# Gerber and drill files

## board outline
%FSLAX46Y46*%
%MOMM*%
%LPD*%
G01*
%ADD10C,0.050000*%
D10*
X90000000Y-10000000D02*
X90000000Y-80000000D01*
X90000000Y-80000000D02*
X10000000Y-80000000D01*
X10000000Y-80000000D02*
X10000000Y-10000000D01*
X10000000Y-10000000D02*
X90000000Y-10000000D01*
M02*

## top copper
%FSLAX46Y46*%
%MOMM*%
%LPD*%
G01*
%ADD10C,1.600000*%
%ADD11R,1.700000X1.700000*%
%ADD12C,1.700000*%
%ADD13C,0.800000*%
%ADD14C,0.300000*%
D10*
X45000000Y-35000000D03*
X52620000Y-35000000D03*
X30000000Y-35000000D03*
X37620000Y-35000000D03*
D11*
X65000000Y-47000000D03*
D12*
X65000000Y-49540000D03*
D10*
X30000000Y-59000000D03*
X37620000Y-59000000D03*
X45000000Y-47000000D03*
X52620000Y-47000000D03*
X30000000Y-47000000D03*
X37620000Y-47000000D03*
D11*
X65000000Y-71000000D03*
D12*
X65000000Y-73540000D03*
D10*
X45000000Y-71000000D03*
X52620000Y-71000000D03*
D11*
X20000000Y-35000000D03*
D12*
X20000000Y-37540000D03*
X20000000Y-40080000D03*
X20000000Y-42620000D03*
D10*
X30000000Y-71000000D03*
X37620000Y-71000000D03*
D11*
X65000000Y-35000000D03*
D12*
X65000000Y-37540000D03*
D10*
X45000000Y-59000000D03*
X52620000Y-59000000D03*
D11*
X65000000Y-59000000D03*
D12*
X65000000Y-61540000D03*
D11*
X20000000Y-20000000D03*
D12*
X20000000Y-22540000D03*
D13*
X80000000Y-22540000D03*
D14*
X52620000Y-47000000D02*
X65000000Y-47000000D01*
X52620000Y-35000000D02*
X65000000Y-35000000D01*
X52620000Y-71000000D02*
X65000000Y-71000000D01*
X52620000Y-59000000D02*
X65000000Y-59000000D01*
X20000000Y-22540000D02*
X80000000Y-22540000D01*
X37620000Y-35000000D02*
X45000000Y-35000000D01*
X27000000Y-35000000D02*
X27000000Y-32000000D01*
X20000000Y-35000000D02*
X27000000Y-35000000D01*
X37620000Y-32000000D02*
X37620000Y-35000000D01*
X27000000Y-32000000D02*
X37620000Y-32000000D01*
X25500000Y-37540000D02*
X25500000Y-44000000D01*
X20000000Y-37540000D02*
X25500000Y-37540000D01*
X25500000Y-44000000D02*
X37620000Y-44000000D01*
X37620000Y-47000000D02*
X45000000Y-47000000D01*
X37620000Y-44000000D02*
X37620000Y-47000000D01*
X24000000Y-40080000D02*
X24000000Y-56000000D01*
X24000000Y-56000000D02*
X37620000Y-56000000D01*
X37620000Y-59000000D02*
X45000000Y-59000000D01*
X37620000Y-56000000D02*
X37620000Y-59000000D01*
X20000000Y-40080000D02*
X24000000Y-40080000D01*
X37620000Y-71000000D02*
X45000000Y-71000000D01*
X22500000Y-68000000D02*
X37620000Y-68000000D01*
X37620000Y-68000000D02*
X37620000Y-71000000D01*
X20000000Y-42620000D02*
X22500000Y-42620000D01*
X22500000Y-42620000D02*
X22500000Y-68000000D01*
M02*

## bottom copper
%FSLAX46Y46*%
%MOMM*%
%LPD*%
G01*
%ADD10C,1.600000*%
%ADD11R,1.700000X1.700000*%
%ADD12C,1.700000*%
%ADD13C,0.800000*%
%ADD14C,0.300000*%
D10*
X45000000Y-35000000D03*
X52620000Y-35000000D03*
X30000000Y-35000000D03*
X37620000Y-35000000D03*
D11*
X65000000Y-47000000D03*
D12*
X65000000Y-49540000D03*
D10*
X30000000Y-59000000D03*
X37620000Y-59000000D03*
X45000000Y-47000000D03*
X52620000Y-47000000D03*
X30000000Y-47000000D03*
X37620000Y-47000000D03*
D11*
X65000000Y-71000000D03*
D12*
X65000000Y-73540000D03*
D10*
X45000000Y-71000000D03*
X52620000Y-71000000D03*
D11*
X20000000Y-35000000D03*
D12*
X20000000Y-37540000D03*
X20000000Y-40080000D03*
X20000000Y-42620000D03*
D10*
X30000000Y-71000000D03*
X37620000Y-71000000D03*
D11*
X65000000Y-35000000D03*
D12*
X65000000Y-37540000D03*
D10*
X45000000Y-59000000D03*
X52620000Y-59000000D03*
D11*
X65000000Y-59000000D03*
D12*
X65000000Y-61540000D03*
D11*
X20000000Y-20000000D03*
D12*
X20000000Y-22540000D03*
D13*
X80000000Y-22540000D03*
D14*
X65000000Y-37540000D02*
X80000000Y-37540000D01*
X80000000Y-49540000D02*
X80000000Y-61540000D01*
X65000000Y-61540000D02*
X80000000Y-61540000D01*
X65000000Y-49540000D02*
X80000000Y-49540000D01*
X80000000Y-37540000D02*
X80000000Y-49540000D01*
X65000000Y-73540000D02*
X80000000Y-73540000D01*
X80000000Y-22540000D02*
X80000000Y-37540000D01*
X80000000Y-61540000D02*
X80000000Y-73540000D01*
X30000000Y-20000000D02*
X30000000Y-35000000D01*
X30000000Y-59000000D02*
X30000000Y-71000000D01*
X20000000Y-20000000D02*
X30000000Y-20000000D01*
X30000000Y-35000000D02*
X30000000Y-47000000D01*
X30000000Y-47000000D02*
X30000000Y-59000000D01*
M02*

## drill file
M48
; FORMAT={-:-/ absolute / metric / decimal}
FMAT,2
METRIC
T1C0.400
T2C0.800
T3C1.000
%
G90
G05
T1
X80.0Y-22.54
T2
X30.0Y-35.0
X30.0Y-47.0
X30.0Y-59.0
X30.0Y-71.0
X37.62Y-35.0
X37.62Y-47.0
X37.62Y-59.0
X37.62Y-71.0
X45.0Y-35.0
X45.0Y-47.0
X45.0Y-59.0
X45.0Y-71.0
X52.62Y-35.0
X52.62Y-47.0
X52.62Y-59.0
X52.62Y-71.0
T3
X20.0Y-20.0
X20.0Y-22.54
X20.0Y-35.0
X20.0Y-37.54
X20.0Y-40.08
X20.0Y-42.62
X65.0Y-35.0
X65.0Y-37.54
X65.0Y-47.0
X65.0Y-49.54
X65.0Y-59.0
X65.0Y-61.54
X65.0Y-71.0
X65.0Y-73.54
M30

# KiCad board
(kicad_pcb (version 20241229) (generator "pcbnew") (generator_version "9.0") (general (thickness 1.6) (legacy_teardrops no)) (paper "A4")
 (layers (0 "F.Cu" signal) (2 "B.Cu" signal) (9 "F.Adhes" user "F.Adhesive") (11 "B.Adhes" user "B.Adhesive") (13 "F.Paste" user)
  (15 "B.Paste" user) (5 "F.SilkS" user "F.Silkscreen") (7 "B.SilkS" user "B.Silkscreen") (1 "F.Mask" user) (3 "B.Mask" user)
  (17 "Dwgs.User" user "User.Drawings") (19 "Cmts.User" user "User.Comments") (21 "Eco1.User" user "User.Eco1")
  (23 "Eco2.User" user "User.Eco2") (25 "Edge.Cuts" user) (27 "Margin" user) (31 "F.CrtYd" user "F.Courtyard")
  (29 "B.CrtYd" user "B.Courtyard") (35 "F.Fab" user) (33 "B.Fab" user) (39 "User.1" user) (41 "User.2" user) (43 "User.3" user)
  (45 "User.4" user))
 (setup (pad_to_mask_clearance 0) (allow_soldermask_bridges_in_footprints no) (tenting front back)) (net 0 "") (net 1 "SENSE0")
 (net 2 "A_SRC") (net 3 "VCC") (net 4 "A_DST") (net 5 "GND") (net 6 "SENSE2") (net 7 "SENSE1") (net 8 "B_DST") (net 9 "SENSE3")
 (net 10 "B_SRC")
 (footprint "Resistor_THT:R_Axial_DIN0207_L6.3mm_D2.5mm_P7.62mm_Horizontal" (layer "F.Cu") (at 45 35)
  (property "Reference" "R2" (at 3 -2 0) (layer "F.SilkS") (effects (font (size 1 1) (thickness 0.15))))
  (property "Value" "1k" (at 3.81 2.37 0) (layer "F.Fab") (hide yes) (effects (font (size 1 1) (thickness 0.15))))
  (pad "1" thru_hole circle (at 0 0) (size 1.6 1.6) (drill 0.8) (layers "*.Cu" "*.Mask") (remove_unused_layers no) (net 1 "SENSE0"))
  (pad "2" thru_hole circle (at 7.62 0) (size 1.6 1.6) (drill 0.8) (layers "*.Cu" "*.Mask") (remove_unused_layers no) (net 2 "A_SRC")))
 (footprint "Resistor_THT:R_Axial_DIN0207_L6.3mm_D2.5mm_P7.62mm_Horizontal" (layer "F.Cu") (at 30 35)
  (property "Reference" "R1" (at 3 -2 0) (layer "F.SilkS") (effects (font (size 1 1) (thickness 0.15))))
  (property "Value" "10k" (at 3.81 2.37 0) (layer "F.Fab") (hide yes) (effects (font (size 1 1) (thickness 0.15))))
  (pad "1" thru_hole circle (at 0 0) (size 1.6 1.6) (drill 0.8) (layers "*.Cu" "*.Mask") (remove_unused_layers no) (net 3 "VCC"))
  (pad "2" thru_hole circle (at 7.62 0) (size 1.6 1.6) (drill 0.8) (layers "*.Cu" "*.Mask") (remove_unused_layers no) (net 1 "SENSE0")))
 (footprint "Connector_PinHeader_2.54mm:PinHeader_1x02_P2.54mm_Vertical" (layer "F.Cu") (at 65 47)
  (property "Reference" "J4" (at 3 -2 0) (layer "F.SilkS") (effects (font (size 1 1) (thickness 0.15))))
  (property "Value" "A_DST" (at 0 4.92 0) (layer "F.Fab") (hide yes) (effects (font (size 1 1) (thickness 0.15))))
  (pad "1" thru_hole rect (at 0 0) (size 1.7 1.7) (drill 1) (layers "*.Cu" "*.Mask") (remove_unused_layers no) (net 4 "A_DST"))
  (pad "2" thru_hole circle (at 0 2.54) (size 1.7 1.7) (drill 1) (layers "*.Cu" "*.Mask") (remove_unused_layers no) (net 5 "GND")))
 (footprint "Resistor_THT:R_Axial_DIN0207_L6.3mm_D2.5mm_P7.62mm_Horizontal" (layer "F.Cu") (at 30 59)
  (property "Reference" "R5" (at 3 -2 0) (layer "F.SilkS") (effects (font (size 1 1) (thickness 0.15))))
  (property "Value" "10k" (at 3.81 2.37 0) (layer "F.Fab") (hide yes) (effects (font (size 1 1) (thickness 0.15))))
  (pad "1" thru_hole circle (at 0 0) (size 1.6 1.6) (drill 0.8) (layers "*.Cu" "*.Mask") (remove_unused_layers no) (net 3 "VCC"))
  (pad "2" thru_hole circle (at 7.62 0) (size 1.6 1.6) (drill 0.8) (layers "*.Cu" "*.Mask") (remove_unused_layers no) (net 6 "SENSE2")))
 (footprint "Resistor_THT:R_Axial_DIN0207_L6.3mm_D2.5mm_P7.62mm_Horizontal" (layer "F.Cu") (at 45 47)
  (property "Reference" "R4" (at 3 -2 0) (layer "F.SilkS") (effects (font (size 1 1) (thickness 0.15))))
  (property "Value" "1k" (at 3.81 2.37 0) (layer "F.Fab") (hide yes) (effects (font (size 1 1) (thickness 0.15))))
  (pad "1" thru_hole circle (at 0 0) (size 1.6 1.6) (drill 0.8) (layers "*.Cu" "*.Mask") (remove_unused_layers no) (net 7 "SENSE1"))
  (pad "2" thru_hole circle (at 7.62 0) (size 1.6 1.6) (drill 0.8) (layers "*.Cu" "*.Mask") (remove_unused_layers no) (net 4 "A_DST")))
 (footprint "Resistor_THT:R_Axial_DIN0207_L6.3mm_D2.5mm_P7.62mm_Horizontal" (layer "F.Cu") (at 30 47)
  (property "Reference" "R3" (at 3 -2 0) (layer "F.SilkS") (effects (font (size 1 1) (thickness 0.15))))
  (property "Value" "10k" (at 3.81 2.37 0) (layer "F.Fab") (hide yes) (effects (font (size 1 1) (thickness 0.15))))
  (pad "1" thru_hole circle (at 0 0) (size 1.6 1.6) (drill 0.8) (layers "*.Cu" "*.Mask") (remove_unused_layers no) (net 3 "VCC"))
  (pad "2" thru_hole circle (at 7.62 0) (size 1.6 1.6) (drill 0.8) (layers "*.Cu" "*.Mask") (remove_unused_layers no) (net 7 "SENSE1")))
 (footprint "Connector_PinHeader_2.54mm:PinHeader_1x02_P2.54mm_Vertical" (layer "F.Cu") (at 65 71)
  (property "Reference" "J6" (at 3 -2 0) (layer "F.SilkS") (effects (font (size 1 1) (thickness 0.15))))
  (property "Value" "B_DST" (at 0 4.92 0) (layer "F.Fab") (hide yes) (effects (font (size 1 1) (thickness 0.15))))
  (pad "1" thru_hole rect (at 0 0) (size 1.7 1.7) (drill 1) (layers "*.Cu" "*.Mask") (remove_unused_layers no) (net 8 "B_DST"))
  (pad "2" thru_hole circle (at 0 2.54) (size 1.7 1.7) (drill 1) (layers "*.Cu" "*.Mask") (remove_unused_layers no) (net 5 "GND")))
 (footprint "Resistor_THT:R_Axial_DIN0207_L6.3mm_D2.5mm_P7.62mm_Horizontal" (layer "F.Cu") (at 45 71)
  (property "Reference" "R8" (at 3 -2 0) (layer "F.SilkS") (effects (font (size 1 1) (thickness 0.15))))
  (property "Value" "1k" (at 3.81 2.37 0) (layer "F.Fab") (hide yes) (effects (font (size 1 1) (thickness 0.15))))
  (pad "1" thru_hole circle (at 0 0) (size 1.6 1.6) (drill 0.8) (layers "*.Cu" "*.Mask") (remove_unused_layers no) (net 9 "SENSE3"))
  (pad "2" thru_hole circle (at 7.62 0) (size 1.6 1.6) (drill 0.8) (layers "*.Cu" "*.Mask") (remove_unused_layers no) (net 8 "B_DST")))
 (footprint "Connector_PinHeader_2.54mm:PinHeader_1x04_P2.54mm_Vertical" (layer "F.Cu") (at 20 35)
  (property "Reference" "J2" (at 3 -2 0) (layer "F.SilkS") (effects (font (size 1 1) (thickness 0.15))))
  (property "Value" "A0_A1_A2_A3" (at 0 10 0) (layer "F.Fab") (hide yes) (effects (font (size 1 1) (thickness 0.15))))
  (pad "1" thru_hole rect (at 0 0) (size 1.7 1.7) (drill 1) (layers "*.Cu" "*.Mask") (remove_unused_layers no) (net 1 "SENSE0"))
  (pad "2" thru_hole circle (at 0 2.54) (size 1.7 1.7) (drill 1) (layers "*.Cu" "*.Mask") (remove_unused_layers no) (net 7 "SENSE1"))
  (pad "3" thru_hole circle (at 0 5.08) (size 1.7 1.7) (drill 1) (layers "*.Cu" "*.Mask") (remove_unused_layers no) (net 6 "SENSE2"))
  (pad "4" thru_hole circle (at 0 7.62) (size 1.7 1.7) (drill 1) (layers "*.Cu" "*.Mask") (remove_unused_layers no) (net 9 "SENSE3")))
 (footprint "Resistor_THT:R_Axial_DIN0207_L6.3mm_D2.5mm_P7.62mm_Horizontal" (layer "F.Cu") (at 30 71)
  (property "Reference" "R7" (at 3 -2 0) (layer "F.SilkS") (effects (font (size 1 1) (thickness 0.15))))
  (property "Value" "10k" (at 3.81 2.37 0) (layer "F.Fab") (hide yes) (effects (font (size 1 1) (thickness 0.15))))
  (pad "1" thru_hole circle (at 0 0) (size 1.6 1.6) (drill 0.8) (layers "*.Cu" "*.Mask") (remove_unused_layers no) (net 3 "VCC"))
  (pad "2" thru_hole circle (at 7.62 0) (size 1.6 1.6) (drill 0.8) (layers "*.Cu" "*.Mask") (remove_unused_layers no) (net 9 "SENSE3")))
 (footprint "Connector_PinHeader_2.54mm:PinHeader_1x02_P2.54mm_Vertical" (layer "F.Cu") (at 65 35)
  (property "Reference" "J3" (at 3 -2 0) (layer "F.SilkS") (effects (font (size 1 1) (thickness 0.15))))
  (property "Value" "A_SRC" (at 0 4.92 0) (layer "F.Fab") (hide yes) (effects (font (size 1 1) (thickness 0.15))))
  (pad "1" thru_hole rect (at 0 0) (size 1.7 1.7) (drill 1) (layers "*.Cu" "*.Mask") (remove_unused_layers no) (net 2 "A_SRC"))
  (pad "2" thru_hole circle (at 0 2.54) (size 1.7 1.7) (drill 1) (layers "*.Cu" "*.Mask") (remove_unused_layers no) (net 5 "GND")))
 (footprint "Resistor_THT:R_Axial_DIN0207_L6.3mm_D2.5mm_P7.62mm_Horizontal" (layer "F.Cu") (at 45 59)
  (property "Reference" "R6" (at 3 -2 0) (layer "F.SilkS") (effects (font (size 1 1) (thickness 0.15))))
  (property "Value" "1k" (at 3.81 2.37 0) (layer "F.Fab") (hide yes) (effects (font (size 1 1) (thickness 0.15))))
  (pad "1" thru_hole circle (at 0 0) (size 1.6 1.6) (drill 0.8) (layers "*.Cu" "*.Mask") (remove_unused_layers no) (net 6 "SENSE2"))
  (pad "2" thru_hole circle (at 7.62 0) (size 1.6 1.6) (drill 0.8) (layers "*.Cu" "*.Mask") (remove_unused_layers no) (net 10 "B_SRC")))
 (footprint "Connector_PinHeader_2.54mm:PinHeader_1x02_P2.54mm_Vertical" (layer "F.Cu") (at 65 59)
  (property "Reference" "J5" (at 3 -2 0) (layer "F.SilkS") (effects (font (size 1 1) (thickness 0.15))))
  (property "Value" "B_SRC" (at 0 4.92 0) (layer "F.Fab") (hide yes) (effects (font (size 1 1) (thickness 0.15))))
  (pad "1" thru_hole rect (at 0 0) (size 1.7 1.7) (drill 1) (layers "*.Cu" "*.Mask") (remove_unused_layers no) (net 10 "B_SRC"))
  (pad "2" thru_hole circle (at 0 2.54) (size 1.7 1.7) (drill 1) (layers "*.Cu" "*.Mask") (remove_unused_layers no) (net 5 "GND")))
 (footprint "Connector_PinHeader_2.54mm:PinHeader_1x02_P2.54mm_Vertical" (layer "F.Cu") (at 20 20)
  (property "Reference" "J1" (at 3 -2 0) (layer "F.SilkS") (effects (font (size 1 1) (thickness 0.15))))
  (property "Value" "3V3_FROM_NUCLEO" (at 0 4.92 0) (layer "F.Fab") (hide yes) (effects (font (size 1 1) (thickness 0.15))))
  (pad "1" thru_hole rect (at 0 0) (size 1.7 1.7) (drill 1) (layers "*.Cu" "*.Mask") (remove_unused_layers no) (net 3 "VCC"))
  (pad "2" thru_hole circle (at 0 2.54) (size 1.7 1.7) (drill 1) (layers "*.Cu" "*.Mask") (remove_unused_layers no) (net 5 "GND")))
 (gr_line (start 90 10) (end 90 80) (stroke (width 0.05) (type default)) (layer "Edge.Cuts"))
 (gr_line (start 90 80) (end 10 80) (stroke (width 0.05) (type default)) (layer "Edge.Cuts"))
 (gr_line (start 10 80) (end 10 10) (stroke (width 0.05) (type default)) (layer "Edge.Cuts"))
 (gr_line (start 10 10) (end 90 10) (stroke (width 0.05) (type default)) (layer "Edge.Cuts"))
 (segment (start 52.62 47) (end 65 47) (width 0.3) (layer "F.Cu") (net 4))
 (segment (start 52.62 35) (end 65 35) (width 0.3) (layer "F.Cu") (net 2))
 (segment (start 52.62 71) (end 65 71) (width 0.3) (layer "F.Cu") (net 8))
 (segment (start 52.62 59) (end 65 59) (width 0.3) (layer "F.Cu") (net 10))
 (segment (start 20 22.54) (end 80 22.54) (width 0.3) (layer "F.Cu") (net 5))
 (via (at 80 22.54) (size 0.8) (drill 0.4) (layers "F.Cu" "B.Cu") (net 5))
 (segment (start 65 37.54) (end 80 37.54) (width 0.3) (layer "B.Cu") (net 5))
 (segment (start 80 49.54) (end 80 61.54) (width 0.3) (layer "B.Cu") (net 5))
 (segment (start 65 61.54) (end 80 61.54) (width 0.3) (layer "B.Cu") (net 5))
 (segment (start 65 49.54) (end 80 49.54) (width 0.3) (layer "B.Cu") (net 5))
 (segment (start 80 37.54) (end 80 49.54) (width 0.3) (layer "B.Cu") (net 5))
 (segment (start 65 73.54) (end 80 73.54) (width 0.3) (layer "B.Cu") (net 5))
 (segment (start 80 22.54) (end 80 37.54) (width 0.3) (layer "B.Cu") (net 5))
 (segment (start 80 61.54) (end 80 73.54) (width 0.3) (layer "B.Cu") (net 5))
 (segment (start 37.62 35) (end 45 35) (width 0.3) (layer "F.Cu") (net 1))
 (segment (start 27 35) (end 27 32) (width 0.3) (layer "F.Cu") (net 1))
 (segment (start 20 35) (end 27 35) (width 0.3) (layer "F.Cu") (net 1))
 (segment (start 37.62 32) (end 37.62 35) (width 0.3) (layer "F.Cu") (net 1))
 (segment (start 27 32) (end 37.62 32) (width 0.3) (layer "F.Cu") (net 1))
 (segment (start 25.5 37.54) (end 25.5 44) (width 0.3) (layer "F.Cu") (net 7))
 (segment (start 20 37.54) (end 25.5 37.54) (width 0.3) (layer "F.Cu") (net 7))
 (segment (start 25.5 44) (end 37.62 44) (width 0.3) (layer "F.Cu") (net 7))
 (segment (start 37.62 47) (end 45 47) (width 0.3) (layer "F.Cu") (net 7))
 (segment (start 37.62 44) (end 37.62 47) (width 0.3) (layer "F.Cu") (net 7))
 (segment (start 24 40.08) (end 24 56) (width 0.3) (layer "F.Cu") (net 6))
 (segment (start 24 56) (end 37.62 56) (width 0.3) (layer "F.Cu") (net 6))
 (segment (start 37.62 59) (end 45 59) (width 0.3) (layer "F.Cu") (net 6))
 (segment (start 37.62 56) (end 37.62 59) (width 0.3) (layer "F.Cu") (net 6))
 (segment (start 20 40.08) (end 24 40.08) (width 0.3) (layer "F.Cu") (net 6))
 (segment (start 37.62 71) (end 45 71) (width 0.3) (layer "F.Cu") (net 9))
 (segment (start 22.5 68) (end 37.62 68) (width 0.3) (layer "F.Cu") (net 9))
 (segment (start 37.62 68) (end 37.62 71) (width 0.3) (layer "F.Cu") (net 9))
 (segment (start 20 42.62) (end 22.5 42.62) (width 0.3) (layer "F.Cu") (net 9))
 (segment (start 22.5 42.62) (end 22.5 68) (width 0.3) (layer "F.Cu") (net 9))
 (segment (start 30 20) (end 30 35) (width 0.3) (layer "B.Cu") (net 3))
 (segment (start 30 59) (end 30 71) (width 0.3) (layer "B.Cu") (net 3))
 (segment (start 20 20) (end 30 20) (width 0.3) (layer "B.Cu") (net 3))
 (segment (start 30 35) (end 30 47) (width 0.3) (layer "B.Cu") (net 3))
 (segment (start 30 47) (end 30 59) (width 0.3) (layer "B.Cu") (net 3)))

